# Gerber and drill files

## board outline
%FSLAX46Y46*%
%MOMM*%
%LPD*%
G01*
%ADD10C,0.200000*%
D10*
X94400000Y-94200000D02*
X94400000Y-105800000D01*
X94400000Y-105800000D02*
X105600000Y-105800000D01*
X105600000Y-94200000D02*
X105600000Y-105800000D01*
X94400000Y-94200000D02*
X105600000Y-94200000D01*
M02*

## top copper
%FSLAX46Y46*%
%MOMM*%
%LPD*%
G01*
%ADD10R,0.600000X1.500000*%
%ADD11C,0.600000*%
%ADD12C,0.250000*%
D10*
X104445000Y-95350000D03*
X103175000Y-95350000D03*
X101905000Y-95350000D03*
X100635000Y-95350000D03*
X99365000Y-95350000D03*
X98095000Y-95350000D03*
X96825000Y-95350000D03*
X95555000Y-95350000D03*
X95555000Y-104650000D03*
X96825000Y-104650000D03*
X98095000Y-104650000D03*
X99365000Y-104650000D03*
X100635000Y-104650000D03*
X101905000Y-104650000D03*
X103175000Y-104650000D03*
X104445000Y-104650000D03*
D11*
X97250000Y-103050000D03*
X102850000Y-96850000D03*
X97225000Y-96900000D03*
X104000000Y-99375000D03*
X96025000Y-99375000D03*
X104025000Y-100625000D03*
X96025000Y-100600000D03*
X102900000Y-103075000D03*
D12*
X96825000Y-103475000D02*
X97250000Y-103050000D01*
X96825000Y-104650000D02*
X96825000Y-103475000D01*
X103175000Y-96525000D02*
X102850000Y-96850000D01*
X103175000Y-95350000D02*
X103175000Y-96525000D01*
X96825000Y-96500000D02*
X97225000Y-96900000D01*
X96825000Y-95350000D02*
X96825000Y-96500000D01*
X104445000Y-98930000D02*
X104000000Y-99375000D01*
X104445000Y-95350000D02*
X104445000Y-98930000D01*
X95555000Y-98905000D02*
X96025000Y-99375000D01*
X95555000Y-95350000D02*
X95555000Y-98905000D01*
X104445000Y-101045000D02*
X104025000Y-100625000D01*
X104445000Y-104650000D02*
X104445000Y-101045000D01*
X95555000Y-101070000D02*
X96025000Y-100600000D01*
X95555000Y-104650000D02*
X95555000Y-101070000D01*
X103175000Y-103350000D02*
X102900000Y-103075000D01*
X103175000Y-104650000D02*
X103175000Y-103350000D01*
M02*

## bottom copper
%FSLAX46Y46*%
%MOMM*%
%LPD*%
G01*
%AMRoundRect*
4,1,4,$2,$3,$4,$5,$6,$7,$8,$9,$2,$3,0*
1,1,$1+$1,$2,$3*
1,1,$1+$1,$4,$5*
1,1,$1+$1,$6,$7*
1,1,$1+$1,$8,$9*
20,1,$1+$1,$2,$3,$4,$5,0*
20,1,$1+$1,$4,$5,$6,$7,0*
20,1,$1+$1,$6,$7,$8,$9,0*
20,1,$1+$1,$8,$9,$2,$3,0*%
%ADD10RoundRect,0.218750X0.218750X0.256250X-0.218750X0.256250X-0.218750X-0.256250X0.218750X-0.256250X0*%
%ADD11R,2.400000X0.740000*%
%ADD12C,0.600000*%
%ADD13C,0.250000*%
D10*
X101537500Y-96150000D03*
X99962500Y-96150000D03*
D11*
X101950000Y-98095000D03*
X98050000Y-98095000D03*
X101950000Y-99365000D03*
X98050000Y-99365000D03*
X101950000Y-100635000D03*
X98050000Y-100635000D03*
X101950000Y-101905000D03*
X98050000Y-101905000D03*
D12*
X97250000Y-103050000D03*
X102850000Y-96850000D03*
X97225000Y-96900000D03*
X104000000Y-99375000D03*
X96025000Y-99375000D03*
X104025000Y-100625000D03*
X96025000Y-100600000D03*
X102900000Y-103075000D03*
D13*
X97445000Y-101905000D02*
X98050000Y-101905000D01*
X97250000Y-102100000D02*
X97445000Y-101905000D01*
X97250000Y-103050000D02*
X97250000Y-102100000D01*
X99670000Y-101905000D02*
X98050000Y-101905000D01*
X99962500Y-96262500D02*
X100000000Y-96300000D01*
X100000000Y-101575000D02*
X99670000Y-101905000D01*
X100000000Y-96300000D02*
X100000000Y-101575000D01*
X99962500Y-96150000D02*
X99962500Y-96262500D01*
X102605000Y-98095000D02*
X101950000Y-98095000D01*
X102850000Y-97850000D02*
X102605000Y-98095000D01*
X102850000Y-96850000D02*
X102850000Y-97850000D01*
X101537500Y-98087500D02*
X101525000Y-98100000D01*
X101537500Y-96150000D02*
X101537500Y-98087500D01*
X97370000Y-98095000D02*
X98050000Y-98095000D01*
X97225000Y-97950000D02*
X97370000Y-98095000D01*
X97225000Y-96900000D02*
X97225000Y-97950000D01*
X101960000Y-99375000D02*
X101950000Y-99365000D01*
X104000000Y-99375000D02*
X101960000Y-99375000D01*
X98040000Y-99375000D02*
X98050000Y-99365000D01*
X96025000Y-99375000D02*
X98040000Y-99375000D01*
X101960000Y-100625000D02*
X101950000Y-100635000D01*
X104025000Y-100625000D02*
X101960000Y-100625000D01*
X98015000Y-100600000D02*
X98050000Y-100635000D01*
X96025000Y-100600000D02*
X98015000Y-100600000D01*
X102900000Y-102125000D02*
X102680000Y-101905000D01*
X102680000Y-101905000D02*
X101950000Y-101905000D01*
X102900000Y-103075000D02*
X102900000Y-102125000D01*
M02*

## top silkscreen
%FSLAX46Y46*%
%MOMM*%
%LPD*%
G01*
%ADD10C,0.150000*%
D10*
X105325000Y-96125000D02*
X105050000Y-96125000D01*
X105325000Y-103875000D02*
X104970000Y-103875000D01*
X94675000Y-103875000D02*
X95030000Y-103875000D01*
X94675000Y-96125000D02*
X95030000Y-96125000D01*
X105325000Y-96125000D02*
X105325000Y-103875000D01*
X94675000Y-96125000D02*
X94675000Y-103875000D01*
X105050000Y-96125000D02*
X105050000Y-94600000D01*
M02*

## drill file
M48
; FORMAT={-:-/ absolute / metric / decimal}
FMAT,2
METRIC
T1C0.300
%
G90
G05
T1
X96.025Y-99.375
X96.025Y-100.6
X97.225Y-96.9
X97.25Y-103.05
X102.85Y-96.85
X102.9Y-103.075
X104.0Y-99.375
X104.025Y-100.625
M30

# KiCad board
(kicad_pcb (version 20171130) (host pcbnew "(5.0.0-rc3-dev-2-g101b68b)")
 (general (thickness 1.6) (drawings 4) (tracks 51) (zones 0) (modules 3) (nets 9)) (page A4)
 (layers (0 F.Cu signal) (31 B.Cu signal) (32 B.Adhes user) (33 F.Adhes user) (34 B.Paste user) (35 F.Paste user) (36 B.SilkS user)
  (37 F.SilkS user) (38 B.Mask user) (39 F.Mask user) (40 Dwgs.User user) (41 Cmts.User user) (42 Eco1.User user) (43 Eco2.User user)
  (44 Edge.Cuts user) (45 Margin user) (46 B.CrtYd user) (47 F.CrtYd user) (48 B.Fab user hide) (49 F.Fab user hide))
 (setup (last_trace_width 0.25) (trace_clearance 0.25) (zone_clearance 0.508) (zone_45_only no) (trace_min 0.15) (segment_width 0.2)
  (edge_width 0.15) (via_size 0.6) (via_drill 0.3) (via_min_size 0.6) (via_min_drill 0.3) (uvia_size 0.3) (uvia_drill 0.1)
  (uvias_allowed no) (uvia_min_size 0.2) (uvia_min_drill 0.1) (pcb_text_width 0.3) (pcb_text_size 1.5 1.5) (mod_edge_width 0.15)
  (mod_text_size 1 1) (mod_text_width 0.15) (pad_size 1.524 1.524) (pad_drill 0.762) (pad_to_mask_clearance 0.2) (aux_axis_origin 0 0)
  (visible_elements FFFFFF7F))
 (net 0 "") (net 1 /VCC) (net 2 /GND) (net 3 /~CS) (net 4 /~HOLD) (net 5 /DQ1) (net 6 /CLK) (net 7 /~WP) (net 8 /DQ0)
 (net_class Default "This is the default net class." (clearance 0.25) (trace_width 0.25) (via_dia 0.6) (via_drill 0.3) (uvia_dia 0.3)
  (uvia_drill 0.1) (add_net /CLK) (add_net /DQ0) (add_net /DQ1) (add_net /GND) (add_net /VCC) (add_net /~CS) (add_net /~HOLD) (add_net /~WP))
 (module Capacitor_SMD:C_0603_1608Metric (layer B.Cu) (at 100.75 96.15 180)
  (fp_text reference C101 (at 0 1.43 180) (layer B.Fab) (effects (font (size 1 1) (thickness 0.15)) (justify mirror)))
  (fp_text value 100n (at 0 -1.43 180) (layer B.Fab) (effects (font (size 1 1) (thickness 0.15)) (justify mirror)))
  (pad 1 smd roundrect (at -0.7875 0 180) (size 0.875 0.95) (layers B.Cu B.Paste B.Mask) (roundrect_rratio 0.25) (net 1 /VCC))
  (pad 2 smd roundrect (at 0.7875 0 180) (size 0.875 0.95) (layers B.Cu B.Paste B.Mask) (roundrect_rratio 0.25) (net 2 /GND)))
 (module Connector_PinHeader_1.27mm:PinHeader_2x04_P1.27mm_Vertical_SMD (layer B.Cu) (at 100 100 180)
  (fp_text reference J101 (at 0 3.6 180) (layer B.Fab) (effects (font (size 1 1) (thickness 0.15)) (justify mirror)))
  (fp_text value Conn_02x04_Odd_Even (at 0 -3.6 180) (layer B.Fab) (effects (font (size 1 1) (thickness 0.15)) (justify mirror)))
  (pad 1 smd rect (at -1.95 1.905 180) (size 2.4 0.74) (layers B.Cu B.Paste B.Mask) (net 1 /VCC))
  (pad 2 smd rect (at 1.95 1.905 180) (size 2.4 0.74) (layers B.Cu B.Paste B.Mask) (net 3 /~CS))
  (pad 3 smd rect (at -1.95 0.635 180) (size 2.4 0.74) (layers B.Cu B.Paste B.Mask) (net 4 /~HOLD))
  (pad 4 smd rect (at 1.95 0.635 180) (size 2.4 0.74) (layers B.Cu B.Paste B.Mask) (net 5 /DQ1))
  (pad 5 smd rect (at -1.95 -0.635 180) (size 2.4 0.74) (layers B.Cu B.Paste B.Mask) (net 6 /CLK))
  (pad 6 smd rect (at 1.95 -0.635 180) (size 2.4 0.74) (layers B.Cu B.Paste B.Mask) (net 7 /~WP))
  (pad 7 smd rect (at -1.95 -1.905 180) (size 2.4 0.74) (layers B.Cu B.Paste B.Mask) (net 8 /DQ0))
  (pad 8 smd rect (at 1.95 -1.905 180) (size 2.4 0.74) (layers B.Cu B.Paste B.Mask) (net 2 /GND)))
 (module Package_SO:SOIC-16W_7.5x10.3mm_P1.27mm (layer F.Cu) (at 100 100 270)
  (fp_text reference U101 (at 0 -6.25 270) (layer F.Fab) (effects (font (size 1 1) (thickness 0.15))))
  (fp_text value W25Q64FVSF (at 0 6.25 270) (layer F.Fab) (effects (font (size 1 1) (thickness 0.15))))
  (fp_line (start -3.875 -5.325) (end -3.875 -5.05) (layer F.SilkS) (width 0.15))
  (fp_line (start 3.875 -5.325) (end 3.875 -4.97) (layer F.SilkS) (width 0.15))
  (fp_line (start 3.875 5.325) (end 3.875 4.97) (layer F.SilkS) (width 0.15))
  (fp_line (start -3.875 5.325) (end -3.875 4.97) (layer F.SilkS) (width 0.15))
  (fp_line (start -3.875 -5.325) (end 3.875 -5.325) (layer F.SilkS) (width 0.15))
  (fp_line (start -3.875 5.325) (end 3.875 5.325) (layer F.SilkS) (width 0.15))
  (fp_line (start -3.875 -5.05) (end -5.4 -5.05) (layer F.SilkS) (width 0.15))
  (pad 1 smd rect (at -4.65 -4.445 270) (size 1.5 0.6) (layers F.Cu F.Paste F.Mask) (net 4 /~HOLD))
  (pad 2 smd rect (at -4.65 -3.175 270) (size 1.5 0.6) (layers F.Cu F.Paste F.Mask) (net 1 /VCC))
  (pad 3 smd rect (at -4.65 -1.905 270) (size 1.5 0.6) (layers F.Cu F.Paste F.Mask))
  (pad 4 smd rect (at -4.65 -0.635 270) (size 1.5 0.6) (layers F.Cu F.Paste F.Mask))
  (pad 5 smd rect (at -4.65 0.635 270) (size 1.5 0.6) (layers F.Cu F.Paste F.Mask))
  (pad 6 smd rect (at -4.65 1.905 270) (size 1.5 0.6) (layers F.Cu F.Paste F.Mask))
  (pad 7 smd rect (at -4.65 3.175 270) (size 1.5 0.6) (layers F.Cu F.Paste F.Mask) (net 3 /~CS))
  (pad 8 smd rect (at -4.65 4.445 270) (size 1.5 0.6) (layers F.Cu F.Paste F.Mask) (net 5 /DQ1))
  (pad 9 smd rect (at 4.65 4.445 270) (size 1.5 0.6) (layers F.Cu F.Paste F.Mask) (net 7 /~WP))
  (pad 10 smd rect (at 4.65 3.175 270) (size 1.5 0.6) (layers F.Cu F.Paste F.Mask) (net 2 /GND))
  (pad 11 smd rect (at 4.65 1.905 270) (size 1.5 0.6) (layers F.Cu F.Paste F.Mask))
  (pad 12 smd rect (at 4.65 0.635 270) (size 1.5 0.6) (layers F.Cu F.Paste F.Mask))
  (pad 13 smd rect (at 4.65 -0.635 270) (size 1.5 0.6) (layers F.Cu F.Paste F.Mask))
  (pad 14 smd rect (at 4.65 -1.905 270) (size 1.5 0.6) (layers F.Cu F.Paste F.Mask))
  (pad 15 smd rect (at 4.65 -3.175 270) (size 1.5 0.6) (layers F.Cu F.Paste F.Mask) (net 8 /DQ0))
  (pad 16 smd rect (at 4.65 -4.445 270) (size 1.5 0.6) (layers F.Cu F.Paste F.Mask) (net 6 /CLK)))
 (gr_line (start 94.4 94.2) (end 94.4 105.8) (layer Edge.Cuts) (width 0.2))
 (gr_line (start 94.4 105.8) (end 105.6 105.8) (layer Edge.Cuts) (width 0.2))
 (gr_line (start 105.6 94.2) (end 105.6 105.8) (layer Edge.Cuts) (width 0.2))
 (gr_line (start 94.4 94.2) (end 105.6 94.2) (layer Edge.Cuts) (width 0.2))
 (via (at 97.25 103.05) (size 0.6) (drill 0.3) (layers F.Cu B.Cu) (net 2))
 (segment (start 96.825 103.475) (end 97.25 103.05) (width 0.25) (layer F.Cu) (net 2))
 (segment (start 96.825 104.65) (end 96.825 103.475) (width 0.25) (layer F.Cu) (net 2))
 (segment (start 97.445 101.905) (end 98.05 101.905) (width 0.25) (layer B.Cu) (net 2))
 (segment (start 97.25 102.1) (end 97.445 101.905) (width 0.25) (layer B.Cu) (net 2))
 (segment (start 97.25 103.05) (end 97.25 102.1) (width 0.25) (layer B.Cu) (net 2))
 (segment (start 99.67 101.905) (end 98.05 101.905) (width 0.25) (layer B.Cu) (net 2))
 (segment (start 99.9625 96.2625) (end 100 96.3) (width 0.25) (layer B.Cu) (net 2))
 (segment (start 100 101.575) (end 99.67 101.905) (width 0.25) (layer B.Cu) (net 2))
 (segment (start 100 96.3) (end 100 101.575) (width 0.25) (layer B.Cu) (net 2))
 (segment (start 99.9625 96.15) (end 99.9625 96.2625) (width 0.25) (layer B.Cu) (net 2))
 (via (at 102.85 96.85) (size 0.6) (drill 0.3) (layers F.Cu B.Cu) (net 1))
 (segment (start 103.175 96.525) (end 102.85 96.85) (width 0.25) (layer F.Cu) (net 1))
 (segment (start 103.175 95.35) (end 103.175 96.525) (width 0.25) (layer F.Cu) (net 1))
 (segment (start 102.605 98.095) (end 101.95 98.095) (width 0.25) (layer B.Cu) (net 1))
 (segment (start 102.85 97.85) (end 102.605 98.095) (width 0.25) (layer B.Cu) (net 1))
 (segment (start 102.85 96.85) (end 102.85 97.85) (width 0.25) (layer B.Cu) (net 1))
 (segment (start 101.5375 98.0875) (end 101.525 98.1) (width 0.25) (layer B.Cu) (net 1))
 (segment (start 101.5375 96.15) (end 101.5375 98.0875) (width 0.25) (layer B.Cu) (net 1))
 (via (at 97.225 96.9) (size 0.6) (drill 0.3) (layers F.Cu B.Cu) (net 3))
 (segment (start 96.825 96.5) (end 97.225 96.9) (width 0.25) (layer F.Cu) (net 3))
 (segment (start 96.825 95.35) (end 96.825 96.5) (width 0.25) (layer F.Cu) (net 3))
 (segment (start 97.37 98.095) (end 98.05 98.095) (width 0.25) (layer B.Cu) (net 3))
 (segment (start 97.225 97.95) (end 97.37 98.095) (width 0.25) (layer B.Cu) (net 3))
 (segment (start 97.225 96.9) (end 97.225 97.95) (width 0.25) (layer B.Cu) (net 3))
 (via (at 104 99.375) (size 0.6) (drill 0.3) (layers F.Cu B.Cu) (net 4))
 (segment (start 104.445 98.93) (end 104 99.375) (width 0.25) (layer F.Cu) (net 4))
 (segment (start 104.445 95.35) (end 104.445 98.93) (width 0.25) (layer F.Cu) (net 4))
 (segment (start 101.96 99.375) (end 101.95 99.365) (width 0.25) (layer B.Cu) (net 4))
 (segment (start 104 99.375) (end 101.96 99.375) (width 0.25) (layer B.Cu) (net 4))
 (via (at 96.025 99.375) (size 0.6) (drill 0.3) (layers F.Cu B.Cu) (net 5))
 (segment (start 95.555 98.905) (end 96.025 99.375) (width 0.25) (layer F.Cu) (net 5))
 (segment (start 95.555 95.35) (end 95.555 98.905) (width 0.25) (layer F.Cu) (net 5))
 (segment (start 98.04 99.375) (end 98.05 99.365) (width 0.25) (layer B.Cu) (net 5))
 (segment (start 96.025 99.375) (end 98.04 99.375) (width 0.25) (layer B.Cu) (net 5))
 (segment (start 104.445 101.045) (end 104.025 100.625) (width 0.25) (layer F.Cu) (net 6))
 (via (at 104.025 100.625) (size 0.6) (drill 0.3) (layers F.Cu B.Cu) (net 6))
 (segment (start 104.445 104.65) (end 104.445 101.045) (width 0.25) (layer F.Cu) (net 6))
 (segment (start 101.96 100.625) (end 101.95 100.635) (width 0.25) (layer B.Cu) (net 6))
 (segment (start 104.025 100.625) (end 101.96 100.625) (width 0.25) (layer B.Cu) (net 6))
 (via (at 96.025 100.6) (size 0.6) (drill 0.3) (layers F.Cu B.Cu) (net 7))
 (segment (start 95.555 101.07) (end 96.025 100.6) (width 0.25) (layer F.Cu) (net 7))
 (segment (start 95.555 104.65) (end 95.555 101.07) (width 0.25) (layer F.Cu) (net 7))
 (segment (start 98.015 100.6) (end 98.05 100.635) (width 0.25) (layer B.Cu) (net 7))
 (segment (start 96.025 100.6) (end 98.015 100.6) (width 0.25) (layer B.Cu) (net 7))
 (via (at 102.9 103.075) (size 0.6) (drill 0.3) (layers F.Cu B.Cu) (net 8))
 (segment (start 103.175 103.35) (end 102.9 103.075) (width 0.25) (layer F.Cu) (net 8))
 (segment (start 103.175 104.65) (end 103.175 103.35) (width 0.25) (layer F.Cu) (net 8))
 (segment (start 102.9 102.125) (end 102.68 101.905) (width 0.25) (layer B.Cu) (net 8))
 (segment (start 102.68 101.905) (end 101.95 101.905) (width 0.25) (layer B.Cu) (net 8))
 (segment (start 102.9 103.075) (end 102.9 102.125) (width 0.25) (layer B.Cu) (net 8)))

